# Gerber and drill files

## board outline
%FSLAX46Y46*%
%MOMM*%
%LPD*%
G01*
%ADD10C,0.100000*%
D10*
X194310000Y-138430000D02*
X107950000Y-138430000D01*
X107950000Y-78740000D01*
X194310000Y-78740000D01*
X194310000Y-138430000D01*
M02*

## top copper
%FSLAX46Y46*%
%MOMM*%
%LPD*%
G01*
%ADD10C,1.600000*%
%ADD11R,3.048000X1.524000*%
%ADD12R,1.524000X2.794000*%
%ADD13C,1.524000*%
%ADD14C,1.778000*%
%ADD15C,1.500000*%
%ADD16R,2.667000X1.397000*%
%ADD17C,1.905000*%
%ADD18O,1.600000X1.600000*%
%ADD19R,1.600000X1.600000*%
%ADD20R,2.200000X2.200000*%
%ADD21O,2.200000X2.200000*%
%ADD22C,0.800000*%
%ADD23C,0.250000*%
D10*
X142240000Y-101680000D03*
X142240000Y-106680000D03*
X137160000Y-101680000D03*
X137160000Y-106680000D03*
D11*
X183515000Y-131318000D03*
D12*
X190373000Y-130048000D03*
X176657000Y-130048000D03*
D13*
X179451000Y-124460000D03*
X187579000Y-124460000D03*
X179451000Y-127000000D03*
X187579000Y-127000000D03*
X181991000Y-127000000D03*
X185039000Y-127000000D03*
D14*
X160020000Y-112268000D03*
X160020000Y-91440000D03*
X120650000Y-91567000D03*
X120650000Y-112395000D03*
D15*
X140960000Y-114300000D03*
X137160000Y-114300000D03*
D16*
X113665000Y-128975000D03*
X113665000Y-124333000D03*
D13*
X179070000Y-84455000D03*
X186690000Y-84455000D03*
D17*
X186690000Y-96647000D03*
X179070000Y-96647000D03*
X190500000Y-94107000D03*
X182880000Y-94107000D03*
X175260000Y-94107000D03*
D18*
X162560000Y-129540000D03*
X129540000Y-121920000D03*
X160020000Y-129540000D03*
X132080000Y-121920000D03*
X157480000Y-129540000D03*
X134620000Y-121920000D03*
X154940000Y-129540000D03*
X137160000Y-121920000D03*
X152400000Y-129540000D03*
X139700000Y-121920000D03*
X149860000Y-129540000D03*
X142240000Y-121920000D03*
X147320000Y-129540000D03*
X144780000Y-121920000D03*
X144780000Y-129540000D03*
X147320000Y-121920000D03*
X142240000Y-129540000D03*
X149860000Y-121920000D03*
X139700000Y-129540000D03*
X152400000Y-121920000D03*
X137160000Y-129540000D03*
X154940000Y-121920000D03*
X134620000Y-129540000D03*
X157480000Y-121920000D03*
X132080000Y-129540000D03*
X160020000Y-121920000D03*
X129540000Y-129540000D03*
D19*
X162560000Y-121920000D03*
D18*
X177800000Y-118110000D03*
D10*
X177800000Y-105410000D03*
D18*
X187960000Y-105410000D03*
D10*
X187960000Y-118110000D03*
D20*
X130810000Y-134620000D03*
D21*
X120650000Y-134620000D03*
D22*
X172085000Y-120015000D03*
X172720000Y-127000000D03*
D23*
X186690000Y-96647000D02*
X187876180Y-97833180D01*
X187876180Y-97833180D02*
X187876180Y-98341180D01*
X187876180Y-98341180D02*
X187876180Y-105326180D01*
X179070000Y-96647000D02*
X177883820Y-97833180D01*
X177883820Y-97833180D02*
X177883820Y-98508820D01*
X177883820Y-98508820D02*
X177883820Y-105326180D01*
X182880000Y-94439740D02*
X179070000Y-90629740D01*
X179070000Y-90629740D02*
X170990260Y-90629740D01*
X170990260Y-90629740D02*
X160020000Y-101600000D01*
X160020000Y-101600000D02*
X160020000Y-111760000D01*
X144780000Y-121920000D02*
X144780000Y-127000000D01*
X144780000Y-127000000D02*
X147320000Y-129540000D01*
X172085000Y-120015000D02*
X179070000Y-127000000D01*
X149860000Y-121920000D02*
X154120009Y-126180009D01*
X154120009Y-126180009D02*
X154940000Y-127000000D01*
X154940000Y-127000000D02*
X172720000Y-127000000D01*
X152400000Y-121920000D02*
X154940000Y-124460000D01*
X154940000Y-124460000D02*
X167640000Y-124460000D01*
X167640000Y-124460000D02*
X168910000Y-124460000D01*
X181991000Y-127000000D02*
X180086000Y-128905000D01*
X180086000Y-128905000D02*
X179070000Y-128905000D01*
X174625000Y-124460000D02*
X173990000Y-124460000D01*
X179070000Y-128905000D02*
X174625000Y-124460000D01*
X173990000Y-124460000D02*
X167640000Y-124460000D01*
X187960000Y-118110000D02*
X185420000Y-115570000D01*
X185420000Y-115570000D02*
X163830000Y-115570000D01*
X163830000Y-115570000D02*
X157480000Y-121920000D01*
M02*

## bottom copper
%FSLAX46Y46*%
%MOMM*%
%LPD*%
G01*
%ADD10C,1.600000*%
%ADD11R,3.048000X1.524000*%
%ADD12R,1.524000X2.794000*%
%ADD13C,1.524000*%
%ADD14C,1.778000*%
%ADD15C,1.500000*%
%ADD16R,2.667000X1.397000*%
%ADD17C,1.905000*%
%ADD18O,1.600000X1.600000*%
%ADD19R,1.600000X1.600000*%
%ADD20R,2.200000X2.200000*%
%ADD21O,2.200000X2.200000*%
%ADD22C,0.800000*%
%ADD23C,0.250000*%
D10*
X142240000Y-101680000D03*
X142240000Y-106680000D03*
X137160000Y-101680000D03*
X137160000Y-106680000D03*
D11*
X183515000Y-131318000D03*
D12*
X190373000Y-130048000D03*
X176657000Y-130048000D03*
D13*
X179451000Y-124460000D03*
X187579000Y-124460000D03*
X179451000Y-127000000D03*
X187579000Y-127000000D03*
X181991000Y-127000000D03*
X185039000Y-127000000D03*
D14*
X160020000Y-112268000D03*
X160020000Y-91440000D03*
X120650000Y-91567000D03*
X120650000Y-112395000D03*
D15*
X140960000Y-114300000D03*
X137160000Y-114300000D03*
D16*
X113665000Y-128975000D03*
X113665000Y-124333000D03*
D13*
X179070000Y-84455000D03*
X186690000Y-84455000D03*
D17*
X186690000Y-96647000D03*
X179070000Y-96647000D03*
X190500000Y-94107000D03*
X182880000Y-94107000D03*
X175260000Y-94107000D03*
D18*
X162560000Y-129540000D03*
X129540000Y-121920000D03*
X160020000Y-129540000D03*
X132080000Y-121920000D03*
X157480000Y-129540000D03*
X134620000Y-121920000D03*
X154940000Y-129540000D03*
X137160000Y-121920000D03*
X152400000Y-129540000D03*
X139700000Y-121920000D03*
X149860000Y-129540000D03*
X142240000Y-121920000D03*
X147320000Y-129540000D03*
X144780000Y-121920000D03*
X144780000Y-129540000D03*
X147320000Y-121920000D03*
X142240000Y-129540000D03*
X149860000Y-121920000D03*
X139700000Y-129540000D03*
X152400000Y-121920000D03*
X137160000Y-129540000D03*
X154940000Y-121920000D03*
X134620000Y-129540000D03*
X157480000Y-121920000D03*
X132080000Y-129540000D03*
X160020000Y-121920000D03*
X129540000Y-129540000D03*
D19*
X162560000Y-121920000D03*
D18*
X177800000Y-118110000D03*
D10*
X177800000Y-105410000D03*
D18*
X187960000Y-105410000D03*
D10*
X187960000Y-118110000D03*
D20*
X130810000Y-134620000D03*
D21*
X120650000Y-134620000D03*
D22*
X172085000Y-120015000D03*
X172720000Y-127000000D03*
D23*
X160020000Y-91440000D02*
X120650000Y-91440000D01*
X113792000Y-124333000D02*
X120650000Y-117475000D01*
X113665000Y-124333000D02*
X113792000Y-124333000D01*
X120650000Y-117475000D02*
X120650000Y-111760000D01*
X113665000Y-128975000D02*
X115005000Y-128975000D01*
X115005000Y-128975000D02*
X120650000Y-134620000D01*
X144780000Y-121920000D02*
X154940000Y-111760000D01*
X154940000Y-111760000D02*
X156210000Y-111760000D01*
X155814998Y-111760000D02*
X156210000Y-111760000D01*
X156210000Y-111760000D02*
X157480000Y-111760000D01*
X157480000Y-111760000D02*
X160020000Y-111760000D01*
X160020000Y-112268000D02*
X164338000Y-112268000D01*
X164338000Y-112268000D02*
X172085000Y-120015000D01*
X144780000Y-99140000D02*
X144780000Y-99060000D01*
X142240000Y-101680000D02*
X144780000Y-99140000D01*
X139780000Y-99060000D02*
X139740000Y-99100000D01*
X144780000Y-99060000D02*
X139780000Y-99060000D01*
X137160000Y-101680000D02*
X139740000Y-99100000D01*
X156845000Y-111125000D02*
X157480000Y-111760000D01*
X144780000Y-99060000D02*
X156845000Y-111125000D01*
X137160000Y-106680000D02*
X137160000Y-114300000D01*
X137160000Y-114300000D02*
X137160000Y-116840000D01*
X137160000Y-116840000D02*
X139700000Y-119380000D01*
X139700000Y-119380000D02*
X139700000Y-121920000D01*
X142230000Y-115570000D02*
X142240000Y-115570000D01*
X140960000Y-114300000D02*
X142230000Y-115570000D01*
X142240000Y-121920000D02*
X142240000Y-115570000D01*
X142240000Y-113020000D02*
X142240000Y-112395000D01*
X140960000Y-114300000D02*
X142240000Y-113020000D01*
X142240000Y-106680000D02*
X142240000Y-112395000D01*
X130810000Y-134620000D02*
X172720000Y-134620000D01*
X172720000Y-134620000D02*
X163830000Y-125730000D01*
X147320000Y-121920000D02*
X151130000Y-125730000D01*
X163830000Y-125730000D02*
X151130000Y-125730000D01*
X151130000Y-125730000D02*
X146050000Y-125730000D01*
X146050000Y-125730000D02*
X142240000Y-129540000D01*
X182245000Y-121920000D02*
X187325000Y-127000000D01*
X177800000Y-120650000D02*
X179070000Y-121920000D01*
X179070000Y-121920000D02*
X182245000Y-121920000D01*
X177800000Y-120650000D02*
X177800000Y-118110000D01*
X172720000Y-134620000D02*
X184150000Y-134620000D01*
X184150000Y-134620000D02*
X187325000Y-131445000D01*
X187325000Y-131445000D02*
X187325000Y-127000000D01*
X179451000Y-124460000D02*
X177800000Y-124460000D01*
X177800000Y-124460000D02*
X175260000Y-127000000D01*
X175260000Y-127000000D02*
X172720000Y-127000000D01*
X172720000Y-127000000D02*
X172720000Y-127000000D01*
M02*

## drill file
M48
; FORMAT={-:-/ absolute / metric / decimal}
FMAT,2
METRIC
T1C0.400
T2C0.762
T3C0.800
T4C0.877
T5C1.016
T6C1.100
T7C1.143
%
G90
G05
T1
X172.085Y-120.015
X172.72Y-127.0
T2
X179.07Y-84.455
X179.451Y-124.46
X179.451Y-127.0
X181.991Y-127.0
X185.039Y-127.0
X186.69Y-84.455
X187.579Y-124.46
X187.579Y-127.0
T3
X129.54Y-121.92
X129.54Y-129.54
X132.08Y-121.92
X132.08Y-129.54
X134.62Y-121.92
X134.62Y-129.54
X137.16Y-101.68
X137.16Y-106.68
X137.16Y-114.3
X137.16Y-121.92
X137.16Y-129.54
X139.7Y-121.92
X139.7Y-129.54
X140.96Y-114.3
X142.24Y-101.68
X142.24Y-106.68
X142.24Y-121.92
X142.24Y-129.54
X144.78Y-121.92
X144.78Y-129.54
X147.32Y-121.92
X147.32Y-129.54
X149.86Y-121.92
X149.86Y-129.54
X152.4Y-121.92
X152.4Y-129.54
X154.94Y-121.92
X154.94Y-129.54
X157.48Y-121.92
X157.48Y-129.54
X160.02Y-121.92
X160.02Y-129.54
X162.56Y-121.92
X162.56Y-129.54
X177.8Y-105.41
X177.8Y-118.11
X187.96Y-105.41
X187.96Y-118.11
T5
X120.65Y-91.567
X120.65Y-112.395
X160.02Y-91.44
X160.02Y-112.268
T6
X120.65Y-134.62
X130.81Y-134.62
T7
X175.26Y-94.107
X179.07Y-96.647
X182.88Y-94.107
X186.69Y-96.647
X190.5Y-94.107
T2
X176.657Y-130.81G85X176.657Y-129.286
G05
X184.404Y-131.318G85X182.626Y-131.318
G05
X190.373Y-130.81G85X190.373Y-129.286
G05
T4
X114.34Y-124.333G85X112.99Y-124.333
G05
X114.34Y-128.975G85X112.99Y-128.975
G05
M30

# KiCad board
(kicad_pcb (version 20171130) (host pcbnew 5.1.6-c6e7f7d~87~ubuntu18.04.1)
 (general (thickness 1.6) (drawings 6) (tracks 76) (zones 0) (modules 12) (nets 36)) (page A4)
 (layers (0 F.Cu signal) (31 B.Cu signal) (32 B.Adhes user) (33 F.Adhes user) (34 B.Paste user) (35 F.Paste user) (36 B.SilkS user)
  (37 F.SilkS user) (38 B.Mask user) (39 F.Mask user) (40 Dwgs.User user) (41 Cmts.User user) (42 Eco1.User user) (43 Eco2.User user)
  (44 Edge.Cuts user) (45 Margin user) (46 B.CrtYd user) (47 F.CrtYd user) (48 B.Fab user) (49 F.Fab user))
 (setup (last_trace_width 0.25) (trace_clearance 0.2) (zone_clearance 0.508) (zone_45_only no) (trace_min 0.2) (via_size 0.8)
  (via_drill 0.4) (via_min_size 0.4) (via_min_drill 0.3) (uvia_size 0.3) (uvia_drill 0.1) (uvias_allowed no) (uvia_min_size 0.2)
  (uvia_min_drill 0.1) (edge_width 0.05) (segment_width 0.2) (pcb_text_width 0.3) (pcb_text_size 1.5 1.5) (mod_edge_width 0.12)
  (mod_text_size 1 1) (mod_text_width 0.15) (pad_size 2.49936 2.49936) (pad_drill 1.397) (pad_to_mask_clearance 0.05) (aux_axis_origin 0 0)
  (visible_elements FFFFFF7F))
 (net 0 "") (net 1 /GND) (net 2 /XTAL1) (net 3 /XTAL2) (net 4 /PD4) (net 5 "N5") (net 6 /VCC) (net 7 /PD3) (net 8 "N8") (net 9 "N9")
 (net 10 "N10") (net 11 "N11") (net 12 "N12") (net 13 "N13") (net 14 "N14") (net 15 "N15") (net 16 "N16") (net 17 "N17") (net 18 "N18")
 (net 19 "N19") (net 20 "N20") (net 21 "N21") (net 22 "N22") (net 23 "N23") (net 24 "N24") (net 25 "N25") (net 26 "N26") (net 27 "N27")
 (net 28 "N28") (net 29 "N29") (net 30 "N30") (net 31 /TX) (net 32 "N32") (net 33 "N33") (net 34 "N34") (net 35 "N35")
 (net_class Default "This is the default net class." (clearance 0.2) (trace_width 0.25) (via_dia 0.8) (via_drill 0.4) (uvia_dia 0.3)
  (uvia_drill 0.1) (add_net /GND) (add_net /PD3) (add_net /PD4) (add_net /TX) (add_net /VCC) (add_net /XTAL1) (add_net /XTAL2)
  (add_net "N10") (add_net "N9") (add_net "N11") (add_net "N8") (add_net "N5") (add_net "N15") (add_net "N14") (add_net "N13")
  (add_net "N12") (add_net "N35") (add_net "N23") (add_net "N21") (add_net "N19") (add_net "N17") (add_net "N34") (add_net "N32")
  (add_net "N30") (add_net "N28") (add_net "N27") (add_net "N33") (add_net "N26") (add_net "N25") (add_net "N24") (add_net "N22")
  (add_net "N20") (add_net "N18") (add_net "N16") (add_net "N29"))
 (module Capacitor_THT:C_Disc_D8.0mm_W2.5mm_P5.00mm (layer F.Cu) (at 142.24 106.68 90)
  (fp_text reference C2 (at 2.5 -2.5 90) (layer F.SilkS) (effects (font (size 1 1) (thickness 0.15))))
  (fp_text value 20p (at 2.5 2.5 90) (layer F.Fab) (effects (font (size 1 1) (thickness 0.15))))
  (pad 2 thru_hole circle (at 5 0 90) (size 1.6 1.6) (drill 0.8) (layers *.Cu *.Mask) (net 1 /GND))
  (pad 1 thru_hole circle (at 0 0 90) (size 1.6 1.6) (drill 0.8) (layers *.Cu *.Mask) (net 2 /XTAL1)))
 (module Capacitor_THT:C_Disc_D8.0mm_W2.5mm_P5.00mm (layer F.Cu) (at 137.16 106.68 90)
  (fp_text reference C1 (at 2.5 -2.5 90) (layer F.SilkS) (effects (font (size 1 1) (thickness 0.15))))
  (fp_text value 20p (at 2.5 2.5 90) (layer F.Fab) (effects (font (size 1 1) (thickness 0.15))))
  (pad 2 thru_hole circle (at 5 0 90) (size 1.6 1.6) (drill 0.8) (layers *.Cu *.Mask) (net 1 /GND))
  (pad 1 thru_hole circle (at 0 0 90) (size 1.6 1.6) (drill 0.8) (layers *.Cu *.Mask) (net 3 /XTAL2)))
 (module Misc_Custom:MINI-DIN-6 (layer F.Cu) (at 183.515 124.46 180)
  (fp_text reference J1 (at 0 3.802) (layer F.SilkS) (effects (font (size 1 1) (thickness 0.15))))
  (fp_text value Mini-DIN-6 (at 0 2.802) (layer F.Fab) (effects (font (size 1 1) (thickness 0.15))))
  (pad "" thru_hole rect (at 0 -6.858 270) (size 1.524 3.048) (drill oval 0.762 2.54) (layers *.Cu *.Mask))
  (pad "" thru_hole rect (at -6.858 -5.588 180) (size 1.524 2.794) (drill oval 0.762 2.286) (layers *.Cu *.Mask))
  (pad "" thru_hole rect (at 6.858 -5.588 180) (size 1.524 2.794) (drill oval 0.762 2.286) (layers *.Cu *.Mask))
  (pad 5 thru_hole circle (at 4.064 0 180) (size 1.524 1.524) (drill 0.762) (layers *.Cu *.Mask) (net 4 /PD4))
  (pad 6 thru_hole circle (at -4.064 0 180) (size 1.524 1.524) (drill 0.762) (layers *.Cu *.Mask) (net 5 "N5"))
  (pad 3 thru_hole circle (at 4.064 -2.54 180) (size 1.524 1.524) (drill 0.762) (layers *.Cu *.Mask) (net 1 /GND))
  (pad 4 thru_hole circle (at -4.064 -2.54 180) (size 1.524 1.524) (drill 0.762) (layers *.Cu *.Mask) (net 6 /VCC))
  (pad 1 thru_hole circle (at 1.524 -2.54 180) (size 1.524 1.524) (drill 0.762) (layers *.Cu *.Mask) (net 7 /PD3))
  (pad 2 thru_hole circle (at -1.524 -2.54 180) (size 1.524 1.524) (drill 0.762) (layers *.Cu *.Mask) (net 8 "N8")))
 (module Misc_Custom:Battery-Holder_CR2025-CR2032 (layer F.Cu) (at 160.02 91.44 180)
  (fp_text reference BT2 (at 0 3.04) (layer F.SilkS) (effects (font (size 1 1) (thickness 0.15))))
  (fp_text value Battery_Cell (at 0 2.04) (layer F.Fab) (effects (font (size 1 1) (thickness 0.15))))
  (pad 2 thru_hole circle (at 0 -20.828 180) (size 1.778 1.778) (drill 1.016) (layers *.Cu *.Mask) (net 1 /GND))
  (pad 1 thru_hole circle (at 0 0 180) (size 1.778 1.778) (drill 1.016) (layers *.Cu *.Mask) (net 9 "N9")))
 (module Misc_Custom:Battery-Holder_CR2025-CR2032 (layer F.Cu) (at 120.65 112.395)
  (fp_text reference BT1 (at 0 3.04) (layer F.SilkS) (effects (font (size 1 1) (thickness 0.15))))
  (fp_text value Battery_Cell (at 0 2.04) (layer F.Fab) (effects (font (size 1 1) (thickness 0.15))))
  (pad 2 thru_hole circle (at 0 -20.828) (size 1.778 1.778) (drill 1.016) (layers *.Cu *.Mask) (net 9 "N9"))
  (pad 1 thru_hole circle (at 0 0) (size 1.778 1.778) (drill 1.016) (layers *.Cu *.Mask) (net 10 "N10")))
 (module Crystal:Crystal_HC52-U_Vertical (layer F.Cu) (at 137.16 114.3)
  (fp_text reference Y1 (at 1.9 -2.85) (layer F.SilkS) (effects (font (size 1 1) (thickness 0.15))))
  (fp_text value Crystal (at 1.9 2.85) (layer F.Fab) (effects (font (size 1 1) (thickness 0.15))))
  (pad 2 thru_hole circle (at 3.8 0) (size 1.5 1.5) (drill 0.8) (layers *.Cu *.Mask) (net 2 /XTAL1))
  (pad 1 thru_hole circle (at 0 0) (size 1.5 1.5) (drill 0.8) (layers *.Cu *.Mask) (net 3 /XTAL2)))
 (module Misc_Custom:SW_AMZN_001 (layer F.Cu) (at 113.665 123.825 180)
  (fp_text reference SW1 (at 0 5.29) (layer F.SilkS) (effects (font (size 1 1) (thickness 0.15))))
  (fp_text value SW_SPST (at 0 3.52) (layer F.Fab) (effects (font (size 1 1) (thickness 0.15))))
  (pad 2 thru_hole rect (at 0 -5.15 270) (size 1.397 2.667) (drill oval 0.877 2.227001) (layers *.Cu *.Mask) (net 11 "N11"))
  (pad 1 thru_hole rect (at 0 -0.508 270) (size 1.397 2.667) (drill oval 0.877 2.227001) (layers *.Cu *.Mask) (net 10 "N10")))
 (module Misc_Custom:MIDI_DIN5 (layer F.Cu) (at 182.88 81.915 180)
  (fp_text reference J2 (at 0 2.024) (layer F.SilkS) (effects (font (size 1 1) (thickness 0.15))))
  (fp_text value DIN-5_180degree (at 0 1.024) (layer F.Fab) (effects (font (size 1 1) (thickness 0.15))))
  (pad "" thru_hole circle (at 3.81 -2.54 180) (size 1.524 1.524) (drill 0.762) (layers *.Cu *.Mask))
  (pad "" thru_hole circle (at -3.81 -2.54 180) (size 1.524 1.524) (drill 0.762) (layers *.Cu *.Mask))
  (pad 5 thru_hole circle (at -3.81 -14.732 180) (size 1.905 1.905) (drill 1.143) (layers *.Cu *.Mask) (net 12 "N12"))
  (pad 4 thru_hole circle (at 3.81 -14.732 180) (size 1.905 1.905) (drill 1.143) (layers *.Cu *.Mask) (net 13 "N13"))
  (pad 3 thru_hole circle (at -7.62 -12.192 180) (size 1.905 1.905) (drill 1.143) (layers *.Cu *.Mask) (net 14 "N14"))
  (pad 2 thru_hole circle (at 0 -12.192 180) (size 1.905 1.905) (drill 1.143) (layers *.Cu *.Mask) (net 1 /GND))
  (pad 1 thru_hole circle (at 7.62 -12.192 180) (size 1.905 1.905) (drill 1.143) (layers *.Cu *.Mask) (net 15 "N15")))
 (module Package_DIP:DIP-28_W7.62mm (layer F.Cu) (at 162.56 121.92 270)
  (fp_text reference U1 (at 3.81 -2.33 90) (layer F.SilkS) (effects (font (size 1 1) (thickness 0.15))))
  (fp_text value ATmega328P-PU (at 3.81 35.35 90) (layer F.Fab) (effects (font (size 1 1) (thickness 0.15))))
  (pad 28 thru_hole oval (at 7.62 0 270) (size 1.6 1.6) (drill 0.8) (layers *.Cu *.Mask) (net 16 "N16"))
  (pad 14 thru_hole oval (at 0 33.02 270) (size 1.6 1.6) (drill 0.8) (layers *.Cu *.Mask) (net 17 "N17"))
  (pad 27 thru_hole oval (at 7.62 2.54 270) (size 1.6 1.6) (drill 0.8) (layers *.Cu *.Mask) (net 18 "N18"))
  (pad 13 thru_hole oval (at 0 30.48 270) (size 1.6 1.6) (drill 0.8) (layers *.Cu *.Mask) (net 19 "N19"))
  (pad 26 thru_hole oval (at 7.62 5.08 270) (size 1.6 1.6) (drill 0.8) (layers *.Cu *.Mask) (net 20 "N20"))
  (pad 12 thru_hole oval (at 0 27.94 270) (size 1.6 1.6) (drill 0.8) (layers *.Cu *.Mask) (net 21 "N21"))
  (pad 25 thru_hole oval (at 7.62 7.62 270) (size 1.6 1.6) (drill 0.8) (layers *.Cu *.Mask) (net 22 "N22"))
  (pad 11 thru_hole oval (at 0 25.4 270) (size 1.6 1.6) (drill 0.8) (layers *.Cu *.Mask) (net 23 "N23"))
  (pad 24 thru_hole oval (at 7.62 10.16 270) (size 1.6 1.6) (drill 0.8) (layers *.Cu *.Mask) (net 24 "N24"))
  (pad 10 thru_hole oval (at 0 22.86 270) (size 1.6 1.6) (drill 0.8) (layers *.Cu *.Mask) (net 3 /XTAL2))
  (pad 23 thru_hole oval (at 7.62 12.7 270) (size 1.6 1.6) (drill 0.8) (layers *.Cu *.Mask) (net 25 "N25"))
  (pad 9 thru_hole oval (at 0 20.32 270) (size 1.6 1.6) (drill 0.8) (layers *.Cu *.Mask) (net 2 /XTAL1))
  (pad 22 thru_hole oval (at 7.62 15.24 270) (size 1.6 1.6) (drill 0.8) (layers *.Cu *.Mask) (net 1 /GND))
  (pad 8 thru_hole oval (at 0 17.78 270) (size 1.6 1.6) (drill 0.8) (layers *.Cu *.Mask) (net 1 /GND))
  (pad 21 thru_hole oval (at 7.62 17.78 270) (size 1.6 1.6) (drill 0.8) (layers *.Cu *.Mask) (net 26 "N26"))
  (pad 7 thru_hole oval (at 0 15.24 270) (size 1.6 1.6) (drill 0.8) (layers *.Cu *.Mask) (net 6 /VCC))
  (pad 20 thru_hole oval (at 7.62 20.32 270) (size 1.6 1.6) (drill 0.8) (layers *.Cu *.Mask) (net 6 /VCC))
  (pad 6 thru_hole oval (at 0 12.7 270) (size 1.6 1.6) (drill 0.8) (layers *.Cu *.Mask) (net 4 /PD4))
  (pad 19 thru_hole oval (at 7.62 22.86 270) (size 1.6 1.6) (drill 0.8) (layers *.Cu *.Mask) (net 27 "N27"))
  (pad 5 thru_hole oval (at 0 10.16 270) (size 1.6 1.6) (drill 0.8) (layers *.Cu *.Mask) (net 7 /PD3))
  (pad 18 thru_hole oval (at 7.62 25.4 270) (size 1.6 1.6) (drill 0.8) (layers *.Cu *.Mask) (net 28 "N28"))
  (pad 4 thru_hole oval (at 0 7.62 270) (size 1.6 1.6) (drill 0.8) (layers *.Cu *.Mask) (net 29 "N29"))
  (pad 17 thru_hole oval (at 7.62 27.94 270) (size 1.6 1.6) (drill 0.8) (layers *.Cu *.Mask) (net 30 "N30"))
  (pad 3 thru_hole oval (at 0 5.08 270) (size 1.6 1.6) (drill 0.8) (layers *.Cu *.Mask) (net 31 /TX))
  (pad 16 thru_hole oval (at 7.62 30.48 270) (size 1.6 1.6) (drill 0.8) (layers *.Cu *.Mask) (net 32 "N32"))
  (pad 2 thru_hole oval (at 0 2.54 270) (size 1.6 1.6) (drill 0.8) (layers *.Cu *.Mask) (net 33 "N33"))
  (pad 15 thru_hole oval (at 7.62 33.02 270) (size 1.6 1.6) (drill 0.8) (layers *.Cu *.Mask) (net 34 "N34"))
  (pad 1 thru_hole rect (at 0 0 270) (size 1.6 1.6) (drill 0.8) (layers *.Cu *.Mask) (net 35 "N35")))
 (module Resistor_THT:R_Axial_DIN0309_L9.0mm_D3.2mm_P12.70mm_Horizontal (layer F.Cu) (at 177.8 105.41 270)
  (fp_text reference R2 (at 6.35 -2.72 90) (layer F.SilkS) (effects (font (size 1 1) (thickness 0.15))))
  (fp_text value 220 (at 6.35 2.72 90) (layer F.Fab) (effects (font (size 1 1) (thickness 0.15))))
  (pad 2 thru_hole oval (at 12.7 0 270) (size 1.6 1.6) (drill 0.8) (layers *.Cu *.Mask) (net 6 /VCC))
  (pad 1 thru_hole circle (at 0 0 270) (size 1.6 1.6) (drill 0.8) (layers *.Cu *.Mask) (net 13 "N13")))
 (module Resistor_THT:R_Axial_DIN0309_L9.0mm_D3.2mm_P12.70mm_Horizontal (layer F.Cu) (at 187.96 118.11 90)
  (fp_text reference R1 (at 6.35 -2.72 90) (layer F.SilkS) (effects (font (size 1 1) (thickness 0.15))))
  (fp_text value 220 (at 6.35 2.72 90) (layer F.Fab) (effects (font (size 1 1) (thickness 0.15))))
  (pad 2 thru_hole oval (at 12.7 0 90) (size 1.6 1.6) (drill 0.8) (layers *.Cu *.Mask) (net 12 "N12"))
  (pad 1 thru_hole circle (at 0 0 90) (size 1.6 1.6) (drill 0.8) (layers *.Cu *.Mask) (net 31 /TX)))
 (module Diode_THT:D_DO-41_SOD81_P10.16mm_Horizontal (layer F.Cu) (at 130.81 134.62 180)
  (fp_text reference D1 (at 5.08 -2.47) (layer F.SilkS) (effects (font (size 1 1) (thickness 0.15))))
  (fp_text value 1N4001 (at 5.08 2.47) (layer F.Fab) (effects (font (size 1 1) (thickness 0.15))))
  (pad 1 thru_hole rect (at 0 0 180) (size 2.2 2.2) (drill 1.1) (layers *.Cu *.Mask) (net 6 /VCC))
  (pad 2 thru_hole oval (at 10.16 0 180) (size 2.2 2.2) (drill 1.1) (layers *.Cu *.Mask) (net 11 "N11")))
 (gr_poly (pts (xy 194.31 138.43) (xy 107.95 138.43) (xy 107.95 78.74) (xy 194.31 78.74)) (layer Edge.Cuts) (width 0.1))
 (segment (start 186.69 96.647) (end 187.87618 97.83318) (width 0.25) (layer F.Cu) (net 12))
 (segment (start 187.87618 97.83318) (end 187.87618 98.34118) (width 0.25) (layer F.Cu) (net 12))
 (segment (start 187.87618 98.34118) (end 187.87618 105.32618) (width 0.25) (layer F.Cu) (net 12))
 (segment (start 179.07 96.647) (end 177.88382 97.83318) (width 0.25) (layer F.Cu) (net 13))
 (segment (start 177.88382 97.83318) (end 177.88382 98.50882) (width 0.25) (layer F.Cu) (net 13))
 (segment (start 177.88382 98.50882) (end 177.88382 105.32618) (width 0.25) (layer F.Cu) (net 13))
 (segment (start 160.02 91.44) (end 120.65 91.44) (width 0.25) (layer B.Cu) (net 9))
 (segment (start 113.792 124.333) (end 120.65 117.475) (width 0.25) (layer B.Cu) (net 10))
 (segment (start 113.665 124.333) (end 113.792 124.333) (width 0.25) (layer B.Cu) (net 10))
 (segment (start 120.65 117.475) (end 120.65 111.76) (width 0.25) (layer B.Cu) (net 10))
 (segment (start 113.665 128.975) (end 115.005 128.975) (width 0.25) (layer B.Cu) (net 11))
 (segment (start 115.005 128.975) (end 120.65 134.62) (width 0.25) (layer B.Cu) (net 11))
 (segment (start 144.78 121.92) (end 154.94 111.76) (width 0.25) (layer B.Cu) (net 1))
 (segment (start 154.94 111.76) (end 156.21 111.76) (width 0.25) (layer B.Cu) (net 1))
 (segment (start 155.814998 111.76) (end 156.21 111.76) (width 0.25) (layer B.Cu) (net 1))
 (segment (start 156.21 111.76) (end 157.48 111.76) (width 0.25) (layer B.Cu) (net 1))
 (segment (start 157.48 111.76) (end 160.02 111.76) (width 0.25) (layer B.Cu) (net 1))
 (segment (start 182.88 94.43974) (end 179.07 90.62974) (width 0.25) (layer F.Cu) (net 1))
 (segment (start 179.07 90.62974) (end 170.99026 90.62974) (width 0.25) (layer F.Cu) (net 1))
 (segment (start 170.99026 90.62974) (end 160.02 101.6) (width 0.25) (layer F.Cu) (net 1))
 (segment (start 160.02 101.6) (end 160.02 111.76) (width 0.25) (layer F.Cu) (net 1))
 (segment (start 144.78 121.92) (end 144.78 127) (width 0.25) (layer F.Cu) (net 1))
 (segment (start 144.78 127) (end 147.32 129.54) (width 0.25) (layer F.Cu) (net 1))
 (segment (start 160.02 112.268) (end 164.338 112.268) (width 0.25) (layer B.Cu) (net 1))
 (segment (start 164.338 112.268) (end 172.085 120.015) (width 0.25) (layer B.Cu) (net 1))
 (via (at 172.085 120.015) (size 0.8) (drill 0.4) (layers F.Cu B.Cu) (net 1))
 (segment (start 172.085 120.015) (end 179.07 127) (width 0.25) (layer F.Cu) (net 1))
 (segment (start 144.78 99.14) (end 144.78 99.06) (width 0.25) (layer B.Cu) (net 1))
 (segment (start 142.24 101.68) (end 144.78 99.14) (width 0.25) (layer B.Cu) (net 1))
 (segment (start 139.78 99.06) (end 139.74 99.1) (width 0.25) (layer B.Cu) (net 1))
 (segment (start 144.78 99.06) (end 139.78 99.06) (width 0.25) (layer B.Cu) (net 1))
 (segment (start 137.16 101.68) (end 139.74 99.1) (width 0.25) (layer B.Cu) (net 1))
 (segment (start 156.845 111.125) (end 157.48 111.76) (width 0.25) (layer B.Cu) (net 1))
 (segment (start 144.78 99.06) (end 156.845 111.125) (width 0.25) (layer B.Cu) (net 1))
 (segment (start 137.16 106.68) (end 137.16 114.3) (width 0.25) (layer B.Cu) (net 3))
 (segment (start 137.16 114.3) (end 137.16 116.84) (width 0.25) (layer B.Cu) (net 3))
 (segment (start 137.16 116.84) (end 139.7 119.38) (width 0.25) (layer B.Cu) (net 3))
 (segment (start 139.7 119.38) (end 139.7 121.92) (width 0.25) (layer B.Cu) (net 3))
 (segment (start 142.23 115.57) (end 142.24 115.57) (width 0.25) (layer B.Cu) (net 2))
 (segment (start 140.96 114.3) (end 142.23 115.57) (width 0.25) (layer B.Cu) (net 2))
 (segment (start 142.24 121.92) (end 142.24 115.57) (width 0.25) (layer B.Cu) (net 2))
 (segment (start 142.24 113.02) (end 142.24 112.395) (width 0.25) (layer B.Cu) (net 2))
 (segment (start 140.96 114.3) (end 142.24 113.02) (width 0.25) (layer B.Cu) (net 2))
 (segment (start 142.24 106.68) (end 142.24 112.395) (width 0.25) (layer B.Cu) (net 2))
 (segment (start 130.81 134.62) (end 172.72 134.62) (width 0.25) (layer B.Cu) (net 6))
 (segment (start 172.72 134.62) (end 163.83 125.73) (width 0.25) (layer B.Cu) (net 6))
 (segment (start 147.32 121.92) (end 151.13 125.73) (width 0.25) (layer B.Cu) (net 6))
 (segment (start 163.83 125.73) (end 151.13 125.73) (width 0.25) (layer B.Cu) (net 6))
 (segment (start 151.13 125.73) (end 146.05 125.73) (width 0.25) (layer B.Cu) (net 6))
 (segment (start 146.05 125.73) (end 142.24 129.54) (width 0.25) (layer B.Cu) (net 6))
 (segment (start 182.245 121.92) (end 187.325 127) (width 0.25) (layer B.Cu) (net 6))
 (segment (start 177.8 120.65) (end 179.07 121.92) (width 0.25) (layer B.Cu) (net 6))
 (segment (start 179.07 121.92) (end 182.245 121.92) (width 0.25) (layer B.Cu) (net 6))
 (segment (start 177.8 120.65) (end 177.8 118.11) (width 0.25) (layer B.Cu) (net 6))
 (segment (start 172.72 134.62) (end 184.15 134.62) (width 0.25) (layer B.Cu) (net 6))
 (segment (start 184.15 134.62) (end 187.325 131.445) (width 0.25) (layer B.Cu) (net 6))
 (segment (start 187.325 131.445) (end 187.325 127) (width 0.25) (layer B.Cu) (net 6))
 (segment (start 149.86 121.92) (end 154.120009 126.180009) (width 0.25) (layer F.Cu) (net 4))
 (segment (start 154.120009 126.180009) (end 154.94 127) (width 0.25) (layer F.Cu) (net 4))
 (segment (start 154.94 127) (end 172.72 127) (width 0.25) (layer F.Cu) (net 4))
 (segment (start 179.451 124.46) (end 177.8 124.46) (width 0.25) (layer B.Cu) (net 4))
 (segment (start 177.8 124.46) (end 175.26 127) (width 0.25) (layer B.Cu) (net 4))
 (segment (start 175.26 127) (end 172.72 127) (width 0.25) (layer B.Cu) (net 4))
 (segment (start 172.72 127) (end 172.72 127) (width 0.25) (layer B.Cu) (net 4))
 (via (at 172.72 127) (size 0.8) (drill 0.4) (layers F.Cu B.Cu) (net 4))
 (segment (start 152.4 121.92) (end 154.94 124.46) (width 0.25) (layer F.Cu) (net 7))
 (segment (start 154.94 124.46) (end 167.64 124.46) (width 0.25) (layer F.Cu) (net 7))
 (segment (start 167.64 124.46) (end 168.91 124.46) (width 0.25) (layer F.Cu) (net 7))
 (segment (start 181.991 127) (end 180.086 128.905) (width 0.25) (layer F.Cu) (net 7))
 (segment (start 180.086 128.905) (end 179.07 128.905) (width 0.25) (layer F.Cu) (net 7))
 (segment (start 174.625 124.46) (end 173.99 124.46) (width 0.25) (layer F.Cu) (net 7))
 (segment (start 179.07 128.905) (end 174.625 124.46) (width 0.25) (layer F.Cu) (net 7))
 (segment (start 173.99 124.46) (end 167.64 124.46) (width 0.25) (layer F.Cu) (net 7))
 (segment (start 187.96 118.11) (end 185.42 115.57) (width 0.25) (layer F.Cu) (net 31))
 (segment (start 185.42 115.57) (end 163.83 115.57) (width 0.25) (layer F.Cu) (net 31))
 (segment (start 163.83 115.57) (end 157.48 121.92) (width 0.25) (layer F.Cu) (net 31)))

